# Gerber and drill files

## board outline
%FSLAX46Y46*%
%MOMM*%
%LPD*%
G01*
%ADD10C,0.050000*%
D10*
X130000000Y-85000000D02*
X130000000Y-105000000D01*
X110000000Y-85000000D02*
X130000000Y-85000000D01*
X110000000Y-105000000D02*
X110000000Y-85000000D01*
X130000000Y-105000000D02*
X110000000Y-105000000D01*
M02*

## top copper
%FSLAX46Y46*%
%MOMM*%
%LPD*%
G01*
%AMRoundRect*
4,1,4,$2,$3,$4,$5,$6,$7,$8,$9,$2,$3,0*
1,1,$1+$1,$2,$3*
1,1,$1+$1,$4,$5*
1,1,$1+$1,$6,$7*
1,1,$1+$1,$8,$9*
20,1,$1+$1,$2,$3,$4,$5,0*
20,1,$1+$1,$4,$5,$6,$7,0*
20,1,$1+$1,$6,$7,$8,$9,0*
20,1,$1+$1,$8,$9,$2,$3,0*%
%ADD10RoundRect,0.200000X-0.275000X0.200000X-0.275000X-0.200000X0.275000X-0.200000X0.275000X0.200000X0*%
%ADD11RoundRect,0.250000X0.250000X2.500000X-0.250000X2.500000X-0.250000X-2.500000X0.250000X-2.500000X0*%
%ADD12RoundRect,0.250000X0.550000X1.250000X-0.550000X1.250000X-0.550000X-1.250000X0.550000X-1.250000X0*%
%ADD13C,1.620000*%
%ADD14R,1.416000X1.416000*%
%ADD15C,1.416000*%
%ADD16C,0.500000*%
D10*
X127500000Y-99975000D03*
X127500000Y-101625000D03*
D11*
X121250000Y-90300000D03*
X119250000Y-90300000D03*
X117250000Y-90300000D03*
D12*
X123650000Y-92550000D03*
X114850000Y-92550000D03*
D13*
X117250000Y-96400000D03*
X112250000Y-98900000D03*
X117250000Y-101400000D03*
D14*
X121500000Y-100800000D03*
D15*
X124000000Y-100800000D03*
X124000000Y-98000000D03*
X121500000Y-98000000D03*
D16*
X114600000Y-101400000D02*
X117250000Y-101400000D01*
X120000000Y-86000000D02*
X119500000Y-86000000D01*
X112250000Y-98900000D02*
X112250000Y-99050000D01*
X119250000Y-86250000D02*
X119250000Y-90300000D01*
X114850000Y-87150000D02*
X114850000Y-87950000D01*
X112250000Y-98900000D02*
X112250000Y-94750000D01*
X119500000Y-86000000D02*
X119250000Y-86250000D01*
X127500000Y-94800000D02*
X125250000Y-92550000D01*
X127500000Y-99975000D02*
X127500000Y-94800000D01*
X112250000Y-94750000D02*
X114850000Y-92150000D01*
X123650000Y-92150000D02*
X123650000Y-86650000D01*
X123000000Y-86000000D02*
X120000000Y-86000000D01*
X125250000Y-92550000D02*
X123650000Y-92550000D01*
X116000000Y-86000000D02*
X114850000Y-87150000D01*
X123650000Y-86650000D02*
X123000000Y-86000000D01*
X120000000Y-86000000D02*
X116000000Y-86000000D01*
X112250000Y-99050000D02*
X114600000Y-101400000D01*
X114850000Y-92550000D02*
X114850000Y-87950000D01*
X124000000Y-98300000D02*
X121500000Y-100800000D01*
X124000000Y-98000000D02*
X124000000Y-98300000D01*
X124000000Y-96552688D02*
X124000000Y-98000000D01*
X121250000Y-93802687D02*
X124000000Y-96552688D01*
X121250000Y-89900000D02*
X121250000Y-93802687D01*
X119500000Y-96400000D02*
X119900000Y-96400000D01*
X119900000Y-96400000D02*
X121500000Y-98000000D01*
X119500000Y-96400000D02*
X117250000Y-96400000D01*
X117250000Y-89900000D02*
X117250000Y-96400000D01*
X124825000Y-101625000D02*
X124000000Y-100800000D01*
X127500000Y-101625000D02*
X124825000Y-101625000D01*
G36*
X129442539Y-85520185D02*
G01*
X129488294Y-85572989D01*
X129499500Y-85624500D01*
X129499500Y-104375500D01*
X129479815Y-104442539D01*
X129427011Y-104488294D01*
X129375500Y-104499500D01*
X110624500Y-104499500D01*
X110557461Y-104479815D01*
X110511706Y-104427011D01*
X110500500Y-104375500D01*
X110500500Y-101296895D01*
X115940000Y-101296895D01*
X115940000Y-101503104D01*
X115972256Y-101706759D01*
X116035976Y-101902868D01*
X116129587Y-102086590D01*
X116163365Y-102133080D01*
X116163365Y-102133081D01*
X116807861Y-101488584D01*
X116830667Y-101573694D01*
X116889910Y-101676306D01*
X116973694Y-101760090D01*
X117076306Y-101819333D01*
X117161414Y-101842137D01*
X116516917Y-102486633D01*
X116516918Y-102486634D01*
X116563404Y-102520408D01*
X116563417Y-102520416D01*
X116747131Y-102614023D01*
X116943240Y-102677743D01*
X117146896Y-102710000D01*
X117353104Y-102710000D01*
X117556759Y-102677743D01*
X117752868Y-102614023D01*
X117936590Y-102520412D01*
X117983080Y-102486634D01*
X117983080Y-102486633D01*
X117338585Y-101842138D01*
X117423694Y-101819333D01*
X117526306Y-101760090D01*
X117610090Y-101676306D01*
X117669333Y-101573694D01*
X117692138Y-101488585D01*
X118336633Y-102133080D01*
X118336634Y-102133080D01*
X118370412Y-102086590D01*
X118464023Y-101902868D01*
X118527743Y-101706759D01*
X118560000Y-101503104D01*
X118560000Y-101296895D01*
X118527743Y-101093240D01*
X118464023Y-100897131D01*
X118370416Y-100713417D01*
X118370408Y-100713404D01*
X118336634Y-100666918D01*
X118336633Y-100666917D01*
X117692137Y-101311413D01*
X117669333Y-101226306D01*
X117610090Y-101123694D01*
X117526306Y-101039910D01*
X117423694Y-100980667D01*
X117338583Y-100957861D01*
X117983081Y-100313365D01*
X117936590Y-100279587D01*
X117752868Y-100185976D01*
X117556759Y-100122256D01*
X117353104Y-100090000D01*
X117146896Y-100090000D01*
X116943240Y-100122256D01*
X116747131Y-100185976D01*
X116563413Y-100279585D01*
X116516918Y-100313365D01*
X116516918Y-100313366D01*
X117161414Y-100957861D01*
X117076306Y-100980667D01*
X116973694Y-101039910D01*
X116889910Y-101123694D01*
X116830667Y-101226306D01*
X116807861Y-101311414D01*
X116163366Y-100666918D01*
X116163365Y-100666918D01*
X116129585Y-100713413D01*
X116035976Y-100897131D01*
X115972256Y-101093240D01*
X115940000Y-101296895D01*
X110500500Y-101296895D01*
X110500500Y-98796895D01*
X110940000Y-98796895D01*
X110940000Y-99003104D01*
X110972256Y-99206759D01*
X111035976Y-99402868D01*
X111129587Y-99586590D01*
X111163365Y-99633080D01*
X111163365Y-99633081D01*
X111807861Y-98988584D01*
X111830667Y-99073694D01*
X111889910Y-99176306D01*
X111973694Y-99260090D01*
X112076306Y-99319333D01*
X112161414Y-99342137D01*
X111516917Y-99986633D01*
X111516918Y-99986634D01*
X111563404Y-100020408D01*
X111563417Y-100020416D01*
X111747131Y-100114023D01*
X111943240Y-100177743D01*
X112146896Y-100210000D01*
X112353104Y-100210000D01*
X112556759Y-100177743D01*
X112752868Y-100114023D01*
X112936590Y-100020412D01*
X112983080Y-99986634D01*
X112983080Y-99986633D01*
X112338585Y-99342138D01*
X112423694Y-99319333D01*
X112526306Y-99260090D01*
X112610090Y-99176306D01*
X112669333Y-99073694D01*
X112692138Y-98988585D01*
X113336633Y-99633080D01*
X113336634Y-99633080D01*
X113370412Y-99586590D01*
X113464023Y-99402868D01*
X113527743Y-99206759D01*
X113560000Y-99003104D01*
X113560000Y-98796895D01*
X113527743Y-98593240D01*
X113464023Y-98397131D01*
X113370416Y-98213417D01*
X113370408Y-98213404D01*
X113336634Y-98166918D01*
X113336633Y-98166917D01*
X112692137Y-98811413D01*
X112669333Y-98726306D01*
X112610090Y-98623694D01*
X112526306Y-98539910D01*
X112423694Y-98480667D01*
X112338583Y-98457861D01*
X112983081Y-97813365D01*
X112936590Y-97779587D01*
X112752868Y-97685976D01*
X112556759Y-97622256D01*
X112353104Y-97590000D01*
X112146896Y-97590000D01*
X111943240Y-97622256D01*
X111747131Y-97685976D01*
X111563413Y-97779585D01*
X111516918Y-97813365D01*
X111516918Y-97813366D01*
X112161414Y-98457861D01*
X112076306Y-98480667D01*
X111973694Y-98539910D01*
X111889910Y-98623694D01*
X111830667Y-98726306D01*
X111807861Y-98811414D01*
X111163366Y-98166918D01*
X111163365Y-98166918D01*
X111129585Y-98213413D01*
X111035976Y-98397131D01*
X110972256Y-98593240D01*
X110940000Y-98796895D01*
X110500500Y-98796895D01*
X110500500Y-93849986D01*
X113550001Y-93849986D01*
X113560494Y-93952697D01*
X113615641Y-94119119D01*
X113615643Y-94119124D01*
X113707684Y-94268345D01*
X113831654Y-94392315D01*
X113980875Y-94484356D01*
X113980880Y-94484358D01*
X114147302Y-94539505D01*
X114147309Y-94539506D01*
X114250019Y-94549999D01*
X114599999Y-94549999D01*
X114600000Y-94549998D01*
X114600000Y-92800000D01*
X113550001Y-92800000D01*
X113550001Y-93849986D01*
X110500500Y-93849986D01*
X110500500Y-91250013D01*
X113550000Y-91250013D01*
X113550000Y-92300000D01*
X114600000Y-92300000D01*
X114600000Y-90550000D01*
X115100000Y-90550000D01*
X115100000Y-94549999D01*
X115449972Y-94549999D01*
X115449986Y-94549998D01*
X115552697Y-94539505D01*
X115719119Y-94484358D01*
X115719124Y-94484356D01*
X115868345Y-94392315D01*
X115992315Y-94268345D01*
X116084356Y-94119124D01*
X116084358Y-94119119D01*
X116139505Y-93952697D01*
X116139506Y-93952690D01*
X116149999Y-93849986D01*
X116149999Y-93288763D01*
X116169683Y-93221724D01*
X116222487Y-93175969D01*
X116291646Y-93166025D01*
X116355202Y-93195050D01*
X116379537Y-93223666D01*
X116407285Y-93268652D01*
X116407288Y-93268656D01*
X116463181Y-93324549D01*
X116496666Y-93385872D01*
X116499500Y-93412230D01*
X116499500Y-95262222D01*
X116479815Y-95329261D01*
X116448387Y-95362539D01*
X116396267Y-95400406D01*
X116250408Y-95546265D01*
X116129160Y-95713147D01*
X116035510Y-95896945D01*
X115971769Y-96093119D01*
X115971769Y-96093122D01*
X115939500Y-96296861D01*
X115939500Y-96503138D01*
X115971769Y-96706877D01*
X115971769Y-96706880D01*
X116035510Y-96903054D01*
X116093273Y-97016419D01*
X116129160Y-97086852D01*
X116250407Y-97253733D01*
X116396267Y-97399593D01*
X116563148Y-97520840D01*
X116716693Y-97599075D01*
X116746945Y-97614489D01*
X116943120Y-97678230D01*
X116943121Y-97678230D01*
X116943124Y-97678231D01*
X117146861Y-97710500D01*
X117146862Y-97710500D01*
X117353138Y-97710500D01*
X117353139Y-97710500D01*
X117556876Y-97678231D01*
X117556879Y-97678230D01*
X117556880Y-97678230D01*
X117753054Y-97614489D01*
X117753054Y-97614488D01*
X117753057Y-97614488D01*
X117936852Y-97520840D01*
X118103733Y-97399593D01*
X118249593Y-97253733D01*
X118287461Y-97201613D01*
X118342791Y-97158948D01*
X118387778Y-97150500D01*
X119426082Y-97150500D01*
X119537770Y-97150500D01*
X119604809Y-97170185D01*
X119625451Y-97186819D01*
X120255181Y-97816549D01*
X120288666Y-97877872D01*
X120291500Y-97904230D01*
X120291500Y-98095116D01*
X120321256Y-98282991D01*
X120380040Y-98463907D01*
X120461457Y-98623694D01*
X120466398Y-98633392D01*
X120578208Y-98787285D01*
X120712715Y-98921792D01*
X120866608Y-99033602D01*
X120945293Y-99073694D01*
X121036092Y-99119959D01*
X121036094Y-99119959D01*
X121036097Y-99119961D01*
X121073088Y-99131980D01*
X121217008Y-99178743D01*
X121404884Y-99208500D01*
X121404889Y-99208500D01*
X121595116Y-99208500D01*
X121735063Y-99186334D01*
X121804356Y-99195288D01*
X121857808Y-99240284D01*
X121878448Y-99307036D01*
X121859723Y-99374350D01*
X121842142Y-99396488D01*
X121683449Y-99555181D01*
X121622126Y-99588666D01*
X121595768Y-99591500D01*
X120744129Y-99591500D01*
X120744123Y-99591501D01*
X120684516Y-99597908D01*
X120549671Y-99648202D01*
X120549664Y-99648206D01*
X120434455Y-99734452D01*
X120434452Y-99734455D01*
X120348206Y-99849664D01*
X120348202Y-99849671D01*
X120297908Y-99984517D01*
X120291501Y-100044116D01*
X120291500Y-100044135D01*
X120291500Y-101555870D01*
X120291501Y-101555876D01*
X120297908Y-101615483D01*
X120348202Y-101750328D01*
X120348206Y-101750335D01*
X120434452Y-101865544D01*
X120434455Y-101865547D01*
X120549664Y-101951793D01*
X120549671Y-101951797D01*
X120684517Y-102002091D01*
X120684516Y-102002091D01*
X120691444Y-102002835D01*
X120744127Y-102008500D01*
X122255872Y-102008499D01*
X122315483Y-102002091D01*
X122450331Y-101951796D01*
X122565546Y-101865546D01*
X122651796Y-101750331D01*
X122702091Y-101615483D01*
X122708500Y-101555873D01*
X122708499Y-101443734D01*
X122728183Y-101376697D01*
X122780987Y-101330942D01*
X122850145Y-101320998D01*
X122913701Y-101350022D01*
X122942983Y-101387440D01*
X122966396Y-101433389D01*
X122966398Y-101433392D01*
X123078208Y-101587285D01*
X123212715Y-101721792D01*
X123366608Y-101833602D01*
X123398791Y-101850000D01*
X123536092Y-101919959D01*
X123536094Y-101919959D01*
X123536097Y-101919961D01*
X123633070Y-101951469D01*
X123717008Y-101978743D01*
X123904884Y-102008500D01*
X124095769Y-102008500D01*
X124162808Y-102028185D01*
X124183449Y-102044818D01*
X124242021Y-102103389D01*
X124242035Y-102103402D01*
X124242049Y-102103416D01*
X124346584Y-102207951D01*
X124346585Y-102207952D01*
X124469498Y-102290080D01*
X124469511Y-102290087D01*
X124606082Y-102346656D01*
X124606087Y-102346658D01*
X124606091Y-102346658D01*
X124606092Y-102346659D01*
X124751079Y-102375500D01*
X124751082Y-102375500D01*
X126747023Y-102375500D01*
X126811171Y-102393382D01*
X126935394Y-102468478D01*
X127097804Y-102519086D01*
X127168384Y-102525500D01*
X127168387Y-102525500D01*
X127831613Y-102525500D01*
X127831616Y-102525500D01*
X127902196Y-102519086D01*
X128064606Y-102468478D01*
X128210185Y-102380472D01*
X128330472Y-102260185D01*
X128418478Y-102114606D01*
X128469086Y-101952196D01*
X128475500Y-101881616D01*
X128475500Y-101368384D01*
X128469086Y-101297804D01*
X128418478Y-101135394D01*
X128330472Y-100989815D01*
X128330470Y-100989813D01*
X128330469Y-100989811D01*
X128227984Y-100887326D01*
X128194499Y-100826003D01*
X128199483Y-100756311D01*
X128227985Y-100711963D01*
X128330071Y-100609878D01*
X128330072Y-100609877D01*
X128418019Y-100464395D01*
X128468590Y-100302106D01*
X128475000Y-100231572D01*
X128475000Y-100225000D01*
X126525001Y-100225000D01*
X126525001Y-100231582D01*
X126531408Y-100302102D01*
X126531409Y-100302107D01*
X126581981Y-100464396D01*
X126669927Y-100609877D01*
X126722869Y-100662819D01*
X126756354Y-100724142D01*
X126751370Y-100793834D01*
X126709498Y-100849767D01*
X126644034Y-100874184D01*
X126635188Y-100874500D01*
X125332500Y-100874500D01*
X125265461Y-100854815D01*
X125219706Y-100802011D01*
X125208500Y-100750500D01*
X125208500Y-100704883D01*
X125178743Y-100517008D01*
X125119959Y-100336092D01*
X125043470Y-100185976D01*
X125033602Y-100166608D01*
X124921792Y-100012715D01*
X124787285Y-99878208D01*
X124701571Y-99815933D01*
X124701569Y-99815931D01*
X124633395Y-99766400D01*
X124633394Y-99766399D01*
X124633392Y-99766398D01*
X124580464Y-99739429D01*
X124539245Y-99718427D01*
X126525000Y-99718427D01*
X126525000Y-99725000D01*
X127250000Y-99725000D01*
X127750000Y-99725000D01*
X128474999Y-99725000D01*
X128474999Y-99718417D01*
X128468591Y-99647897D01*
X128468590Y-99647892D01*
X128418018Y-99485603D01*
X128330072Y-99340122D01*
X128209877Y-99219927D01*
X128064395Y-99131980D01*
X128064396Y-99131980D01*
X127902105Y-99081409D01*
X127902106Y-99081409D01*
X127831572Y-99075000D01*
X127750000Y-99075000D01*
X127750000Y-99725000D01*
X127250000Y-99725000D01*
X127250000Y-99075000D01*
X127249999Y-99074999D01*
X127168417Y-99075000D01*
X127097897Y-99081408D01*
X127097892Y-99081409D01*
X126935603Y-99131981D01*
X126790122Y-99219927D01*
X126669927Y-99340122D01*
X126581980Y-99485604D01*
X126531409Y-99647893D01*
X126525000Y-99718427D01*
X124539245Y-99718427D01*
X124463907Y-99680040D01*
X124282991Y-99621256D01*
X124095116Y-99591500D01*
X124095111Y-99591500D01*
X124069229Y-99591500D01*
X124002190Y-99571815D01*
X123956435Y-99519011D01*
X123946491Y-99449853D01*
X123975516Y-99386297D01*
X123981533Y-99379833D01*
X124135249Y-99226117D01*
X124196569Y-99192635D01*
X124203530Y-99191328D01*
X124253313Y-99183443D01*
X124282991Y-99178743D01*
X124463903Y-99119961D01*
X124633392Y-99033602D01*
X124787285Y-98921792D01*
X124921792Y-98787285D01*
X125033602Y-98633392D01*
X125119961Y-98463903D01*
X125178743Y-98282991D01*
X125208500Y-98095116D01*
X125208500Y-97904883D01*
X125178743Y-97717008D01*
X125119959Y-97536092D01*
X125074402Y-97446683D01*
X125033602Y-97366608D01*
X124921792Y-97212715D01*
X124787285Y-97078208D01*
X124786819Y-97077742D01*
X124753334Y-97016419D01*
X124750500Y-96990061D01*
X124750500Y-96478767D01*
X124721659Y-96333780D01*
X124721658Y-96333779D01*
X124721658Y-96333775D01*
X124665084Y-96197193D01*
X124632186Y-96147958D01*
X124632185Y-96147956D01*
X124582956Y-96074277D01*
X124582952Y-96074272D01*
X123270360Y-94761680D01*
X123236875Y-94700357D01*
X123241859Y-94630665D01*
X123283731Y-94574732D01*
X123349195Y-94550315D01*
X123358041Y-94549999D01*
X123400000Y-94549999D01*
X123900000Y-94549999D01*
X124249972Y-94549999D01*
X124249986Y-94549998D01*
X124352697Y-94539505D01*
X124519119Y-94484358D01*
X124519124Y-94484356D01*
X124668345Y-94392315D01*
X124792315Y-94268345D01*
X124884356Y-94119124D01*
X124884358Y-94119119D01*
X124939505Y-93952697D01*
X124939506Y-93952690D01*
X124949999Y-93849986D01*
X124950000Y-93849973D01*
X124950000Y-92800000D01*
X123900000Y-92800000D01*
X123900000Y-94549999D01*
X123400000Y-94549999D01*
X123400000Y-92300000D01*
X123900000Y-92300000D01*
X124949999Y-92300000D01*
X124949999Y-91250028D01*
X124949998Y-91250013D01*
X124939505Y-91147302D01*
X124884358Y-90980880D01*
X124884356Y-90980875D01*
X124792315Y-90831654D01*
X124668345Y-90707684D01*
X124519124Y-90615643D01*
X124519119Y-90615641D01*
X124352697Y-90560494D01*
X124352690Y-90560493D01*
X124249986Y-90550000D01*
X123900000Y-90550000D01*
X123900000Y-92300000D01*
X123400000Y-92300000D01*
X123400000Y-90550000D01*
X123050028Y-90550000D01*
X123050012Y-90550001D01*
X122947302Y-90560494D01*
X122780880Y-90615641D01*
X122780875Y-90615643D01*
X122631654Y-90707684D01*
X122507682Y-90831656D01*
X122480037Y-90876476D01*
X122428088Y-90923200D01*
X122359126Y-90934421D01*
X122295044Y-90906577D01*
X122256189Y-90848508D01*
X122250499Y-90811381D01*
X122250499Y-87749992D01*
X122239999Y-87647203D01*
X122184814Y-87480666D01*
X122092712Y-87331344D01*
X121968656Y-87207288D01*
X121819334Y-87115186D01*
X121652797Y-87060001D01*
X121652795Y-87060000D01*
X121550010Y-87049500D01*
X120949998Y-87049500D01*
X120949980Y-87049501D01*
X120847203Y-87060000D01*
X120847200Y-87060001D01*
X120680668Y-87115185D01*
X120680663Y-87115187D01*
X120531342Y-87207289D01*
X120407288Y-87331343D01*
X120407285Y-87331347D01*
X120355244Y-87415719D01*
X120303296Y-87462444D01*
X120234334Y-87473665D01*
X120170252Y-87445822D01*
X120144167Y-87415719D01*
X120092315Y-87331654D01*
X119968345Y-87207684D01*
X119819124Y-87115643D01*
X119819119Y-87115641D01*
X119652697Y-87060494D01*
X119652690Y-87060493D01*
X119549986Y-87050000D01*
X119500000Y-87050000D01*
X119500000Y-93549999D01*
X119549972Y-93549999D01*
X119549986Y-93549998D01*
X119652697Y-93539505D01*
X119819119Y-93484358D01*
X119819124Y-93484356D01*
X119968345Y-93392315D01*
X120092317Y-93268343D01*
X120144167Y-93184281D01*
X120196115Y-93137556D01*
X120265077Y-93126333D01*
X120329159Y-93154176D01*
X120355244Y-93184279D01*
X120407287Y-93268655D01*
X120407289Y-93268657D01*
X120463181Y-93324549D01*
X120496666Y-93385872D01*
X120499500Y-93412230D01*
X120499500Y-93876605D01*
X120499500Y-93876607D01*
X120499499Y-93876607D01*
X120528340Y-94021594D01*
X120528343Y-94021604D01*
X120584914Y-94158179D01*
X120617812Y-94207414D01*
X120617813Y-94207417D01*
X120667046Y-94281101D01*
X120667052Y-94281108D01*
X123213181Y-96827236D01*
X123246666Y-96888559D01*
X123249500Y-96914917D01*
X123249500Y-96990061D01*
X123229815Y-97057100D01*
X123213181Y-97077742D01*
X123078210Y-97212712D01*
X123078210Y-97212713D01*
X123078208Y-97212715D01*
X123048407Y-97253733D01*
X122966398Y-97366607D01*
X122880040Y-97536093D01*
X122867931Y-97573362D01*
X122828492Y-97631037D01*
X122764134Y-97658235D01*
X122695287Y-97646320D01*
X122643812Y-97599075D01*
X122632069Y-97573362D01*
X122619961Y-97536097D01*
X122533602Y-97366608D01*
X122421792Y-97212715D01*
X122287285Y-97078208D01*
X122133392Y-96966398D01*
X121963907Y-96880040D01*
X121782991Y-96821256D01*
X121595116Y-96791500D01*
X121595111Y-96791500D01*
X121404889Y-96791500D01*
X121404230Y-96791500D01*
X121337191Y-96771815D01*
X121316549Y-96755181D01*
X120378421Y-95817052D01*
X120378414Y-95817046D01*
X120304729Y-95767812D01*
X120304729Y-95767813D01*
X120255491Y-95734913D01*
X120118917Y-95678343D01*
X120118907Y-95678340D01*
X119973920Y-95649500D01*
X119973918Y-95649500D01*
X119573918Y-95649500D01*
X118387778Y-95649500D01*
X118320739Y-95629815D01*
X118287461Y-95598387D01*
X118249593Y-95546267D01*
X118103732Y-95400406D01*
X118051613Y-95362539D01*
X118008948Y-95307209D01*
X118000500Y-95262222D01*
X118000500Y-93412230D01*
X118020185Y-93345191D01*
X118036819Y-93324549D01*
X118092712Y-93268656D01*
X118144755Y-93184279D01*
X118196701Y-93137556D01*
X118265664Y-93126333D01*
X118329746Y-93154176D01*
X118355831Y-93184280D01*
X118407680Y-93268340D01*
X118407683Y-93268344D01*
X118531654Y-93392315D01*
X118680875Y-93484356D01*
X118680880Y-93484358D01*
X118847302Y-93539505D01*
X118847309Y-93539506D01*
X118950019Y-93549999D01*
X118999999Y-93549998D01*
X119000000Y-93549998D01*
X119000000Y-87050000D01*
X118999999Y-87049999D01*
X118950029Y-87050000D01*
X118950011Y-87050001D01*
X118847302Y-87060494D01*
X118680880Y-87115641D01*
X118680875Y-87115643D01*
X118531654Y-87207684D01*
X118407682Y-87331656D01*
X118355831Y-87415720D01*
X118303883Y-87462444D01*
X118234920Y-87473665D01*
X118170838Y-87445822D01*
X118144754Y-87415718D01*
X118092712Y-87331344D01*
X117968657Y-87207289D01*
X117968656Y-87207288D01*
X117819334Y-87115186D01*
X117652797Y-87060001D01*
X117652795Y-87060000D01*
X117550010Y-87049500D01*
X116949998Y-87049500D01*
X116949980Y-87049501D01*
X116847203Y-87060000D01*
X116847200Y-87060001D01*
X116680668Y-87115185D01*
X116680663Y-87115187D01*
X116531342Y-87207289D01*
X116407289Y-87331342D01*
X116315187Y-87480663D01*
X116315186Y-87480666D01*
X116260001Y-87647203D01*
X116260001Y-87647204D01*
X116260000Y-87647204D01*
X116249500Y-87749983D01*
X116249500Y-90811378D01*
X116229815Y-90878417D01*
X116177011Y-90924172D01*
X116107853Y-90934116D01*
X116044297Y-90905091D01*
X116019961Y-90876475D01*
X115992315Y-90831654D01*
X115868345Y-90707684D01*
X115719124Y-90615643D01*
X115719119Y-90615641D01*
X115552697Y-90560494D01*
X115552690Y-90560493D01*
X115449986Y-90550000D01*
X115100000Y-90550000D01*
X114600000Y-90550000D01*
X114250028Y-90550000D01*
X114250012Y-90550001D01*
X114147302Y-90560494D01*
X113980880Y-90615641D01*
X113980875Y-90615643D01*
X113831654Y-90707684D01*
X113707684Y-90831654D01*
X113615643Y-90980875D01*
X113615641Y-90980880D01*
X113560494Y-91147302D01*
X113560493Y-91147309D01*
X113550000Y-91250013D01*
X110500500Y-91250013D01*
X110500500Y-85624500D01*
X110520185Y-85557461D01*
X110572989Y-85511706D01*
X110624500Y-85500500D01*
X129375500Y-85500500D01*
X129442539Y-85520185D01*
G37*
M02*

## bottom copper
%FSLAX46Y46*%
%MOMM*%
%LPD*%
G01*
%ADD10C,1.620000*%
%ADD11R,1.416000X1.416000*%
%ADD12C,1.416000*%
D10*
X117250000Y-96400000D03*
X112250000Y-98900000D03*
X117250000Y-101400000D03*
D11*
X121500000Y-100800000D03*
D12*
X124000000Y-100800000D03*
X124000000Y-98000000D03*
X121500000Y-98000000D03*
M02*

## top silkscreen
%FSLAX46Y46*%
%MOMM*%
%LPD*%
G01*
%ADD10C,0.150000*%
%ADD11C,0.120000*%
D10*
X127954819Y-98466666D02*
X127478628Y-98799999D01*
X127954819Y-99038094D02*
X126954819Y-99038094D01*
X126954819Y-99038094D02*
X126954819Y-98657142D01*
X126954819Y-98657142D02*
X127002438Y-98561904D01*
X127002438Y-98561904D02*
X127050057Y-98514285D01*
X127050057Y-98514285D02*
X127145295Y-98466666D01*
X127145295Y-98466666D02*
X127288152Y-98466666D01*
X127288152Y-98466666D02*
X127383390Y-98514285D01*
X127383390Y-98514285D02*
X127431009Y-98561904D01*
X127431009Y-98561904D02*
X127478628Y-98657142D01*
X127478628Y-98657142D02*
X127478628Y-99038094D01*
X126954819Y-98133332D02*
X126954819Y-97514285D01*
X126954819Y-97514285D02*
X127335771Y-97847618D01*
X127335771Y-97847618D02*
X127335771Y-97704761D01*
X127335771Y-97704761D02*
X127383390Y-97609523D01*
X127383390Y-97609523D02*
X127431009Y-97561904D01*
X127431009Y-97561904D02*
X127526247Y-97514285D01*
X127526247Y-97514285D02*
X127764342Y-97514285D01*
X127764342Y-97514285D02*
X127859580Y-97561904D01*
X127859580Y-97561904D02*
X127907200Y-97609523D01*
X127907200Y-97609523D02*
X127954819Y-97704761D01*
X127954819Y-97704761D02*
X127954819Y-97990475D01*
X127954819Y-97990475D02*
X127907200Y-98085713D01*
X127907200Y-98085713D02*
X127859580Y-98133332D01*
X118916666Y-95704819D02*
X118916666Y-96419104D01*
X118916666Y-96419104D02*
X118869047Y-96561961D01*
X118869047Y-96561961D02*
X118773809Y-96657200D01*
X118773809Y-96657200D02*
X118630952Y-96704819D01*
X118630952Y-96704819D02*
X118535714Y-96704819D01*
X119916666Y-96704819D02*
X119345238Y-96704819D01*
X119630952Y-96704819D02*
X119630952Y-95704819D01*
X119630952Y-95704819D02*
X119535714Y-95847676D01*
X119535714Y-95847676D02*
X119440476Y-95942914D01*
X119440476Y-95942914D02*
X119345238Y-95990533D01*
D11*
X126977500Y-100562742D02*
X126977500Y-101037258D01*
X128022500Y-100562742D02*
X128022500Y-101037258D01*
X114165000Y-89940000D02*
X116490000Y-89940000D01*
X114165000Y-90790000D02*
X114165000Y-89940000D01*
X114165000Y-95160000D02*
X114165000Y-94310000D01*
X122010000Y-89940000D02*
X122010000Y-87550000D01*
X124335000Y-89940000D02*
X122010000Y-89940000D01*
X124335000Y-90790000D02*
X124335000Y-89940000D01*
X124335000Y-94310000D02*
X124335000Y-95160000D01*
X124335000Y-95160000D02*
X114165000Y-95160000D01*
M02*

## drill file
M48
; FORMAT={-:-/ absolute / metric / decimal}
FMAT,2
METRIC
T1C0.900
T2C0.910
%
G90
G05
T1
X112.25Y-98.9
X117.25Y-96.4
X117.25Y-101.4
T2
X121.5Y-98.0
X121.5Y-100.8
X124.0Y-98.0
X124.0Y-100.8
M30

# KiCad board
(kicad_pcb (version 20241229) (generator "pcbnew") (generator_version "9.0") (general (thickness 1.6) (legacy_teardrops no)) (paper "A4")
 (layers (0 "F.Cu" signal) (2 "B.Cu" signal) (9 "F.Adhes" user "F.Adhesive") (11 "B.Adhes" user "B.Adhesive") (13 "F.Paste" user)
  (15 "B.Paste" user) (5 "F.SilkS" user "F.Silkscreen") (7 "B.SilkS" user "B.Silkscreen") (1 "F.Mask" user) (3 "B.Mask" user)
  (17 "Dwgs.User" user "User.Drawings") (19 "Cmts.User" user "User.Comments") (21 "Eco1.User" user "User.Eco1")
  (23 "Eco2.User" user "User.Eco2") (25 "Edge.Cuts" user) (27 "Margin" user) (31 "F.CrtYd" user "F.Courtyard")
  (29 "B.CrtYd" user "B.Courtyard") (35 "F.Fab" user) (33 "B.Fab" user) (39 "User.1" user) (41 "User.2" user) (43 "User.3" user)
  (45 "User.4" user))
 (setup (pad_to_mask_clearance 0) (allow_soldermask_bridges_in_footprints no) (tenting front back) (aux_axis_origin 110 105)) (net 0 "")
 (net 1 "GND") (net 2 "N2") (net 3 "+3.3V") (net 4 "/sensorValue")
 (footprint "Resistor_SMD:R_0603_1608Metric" (layer "F.Cu") (at 127.5 100.8 -90)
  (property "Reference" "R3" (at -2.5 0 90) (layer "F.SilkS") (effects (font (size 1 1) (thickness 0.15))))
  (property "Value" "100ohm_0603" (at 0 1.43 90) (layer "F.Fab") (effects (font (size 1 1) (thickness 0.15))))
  (fp_line (start -0.237258 0.5225) (end 0.237258 0.5225) (stroke (width 0.12) (type solid)) (layer "F.SilkS"))
  (fp_line (start -0.237258 -0.5225) (end 0.237258 -0.5225) (stroke (width 0.12) (type solid)) (layer "F.SilkS"))
  (pad "1" smd roundrect (at -0.825 0 270) (size 0.8 0.95) (layers "F.Cu" "F.Mask" "F.Paste") (roundrect_rratio 0.25) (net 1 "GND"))
  (pad "2" smd roundrect (at 0.825 0 270) (size 0.8 0.95) (layers "F.Cu" "F.Mask" "F.Paste") (roundrect_rratio 0.25) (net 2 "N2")))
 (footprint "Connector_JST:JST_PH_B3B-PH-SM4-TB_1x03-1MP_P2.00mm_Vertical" (layer "F.Cu") (at 119.25 90.8 180)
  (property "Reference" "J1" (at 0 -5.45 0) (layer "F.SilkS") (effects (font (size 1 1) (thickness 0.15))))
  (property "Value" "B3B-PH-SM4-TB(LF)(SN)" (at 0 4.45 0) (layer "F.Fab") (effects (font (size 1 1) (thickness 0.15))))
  (fp_line (start 5.085 0.86) (end 2.76 0.86) (stroke (width 0.12) (type solid)) (layer "F.SilkS"))
  (fp_line (start 5.085 0.01) (end 5.085 0.86) (stroke (width 0.12) (type solid)) (layer "F.SilkS"))
  (fp_line (start 5.085 -4.36) (end 5.085 -3.51) (stroke (width 0.12) (type solid)) (layer "F.SilkS"))
  (fp_line (start -2.76 0.86) (end -2.76 3.25) (stroke (width 0.12) (type solid)) (layer "F.SilkS"))
  (fp_line (start -5.085 0.86) (end -2.76 0.86) (stroke (width 0.12) (type solid)) (layer "F.SilkS"))
  (fp_line (start -5.085 0.01) (end -5.085 0.86) (stroke (width 0.12) (type solid)) (layer "F.SilkS"))
  (fp_line (start -5.085 -3.51) (end -5.085 -4.36) (stroke (width 0.12) (type solid)) (layer "F.SilkS"))
  (fp_line (start -5.085 -4.36) (end 5.085 -4.36) (stroke (width 0.12) (type solid)) (layer "F.SilkS"))
  (pad "1" smd roundrect (at -2 0.5 180) (size 1 5.5) (layers "F.Cu" "F.Mask" "F.Paste") (roundrect_rratio 0.25) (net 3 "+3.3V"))
  (pad "2" smd roundrect (at 0 0.5 180) (size 1 5.5) (layers "F.Cu" "F.Mask" "F.Paste") (roundrect_rratio 0.25) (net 1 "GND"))
  (pad "3" smd roundrect (at 2 0.5 180) (size 1 5.5) (layers "F.Cu" "F.Mask" "F.Paste") (roundrect_rratio 0.25) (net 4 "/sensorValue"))
  (pad "MP" smd roundrect (at -4.4 -1.75 180) (size 1.6 3) (layers "F.Cu" "F.Mask" "F.Paste") (roundrect_rratio 0.15625) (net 1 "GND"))
  (pad "MP" smd roundrect (at 4.4 -1.75 180) (size 1.6 3) (layers "F.Cu" "F.Mask" "F.Paste") (roundrect_rratio 0.15625) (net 1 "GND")))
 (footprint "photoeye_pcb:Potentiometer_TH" (layer "B.Cu") (at 117.25 96.4 180)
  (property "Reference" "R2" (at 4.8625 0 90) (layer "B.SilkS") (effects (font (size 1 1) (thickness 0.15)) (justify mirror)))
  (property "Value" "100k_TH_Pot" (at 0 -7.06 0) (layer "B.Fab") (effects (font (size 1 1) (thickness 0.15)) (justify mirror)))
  (pad "1" thru_hole circle (at 0 0 180) (size 1.62 1.62) (drill 0.9) (layers "*.Cu" "*.Mask") (remove_unused_layers no)
   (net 4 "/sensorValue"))
  (pad "2" thru_hole circle (at 5 -2.5 180) (size 1.62 1.62) (drill 0.9) (layers "*.Cu" "*.Mask") (remove_unused_layers no) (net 1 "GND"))
  (pad "3" thru_hole circle (at 0 -5 180) (size 1.62 1.62) (drill 0.9) (layers "*.Cu" "*.Mask") (remove_unused_layers no) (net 1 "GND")))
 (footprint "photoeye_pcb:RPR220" (layer "B.Cu") (at 121.5 100.8 90)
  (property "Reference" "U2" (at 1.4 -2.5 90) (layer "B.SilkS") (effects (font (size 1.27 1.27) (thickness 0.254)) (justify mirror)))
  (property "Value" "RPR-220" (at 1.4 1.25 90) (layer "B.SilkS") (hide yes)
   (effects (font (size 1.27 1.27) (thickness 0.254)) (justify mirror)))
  (pad "1" thru_hole rect (at 0 0 90) (size 1.416 1.416) (drill 0.91) (layers "*.Cu" "*.Mask") (remove_unused_layers no) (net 3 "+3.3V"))
  (pad "2" thru_hole circle (at 0 2.5 90) (size 1.416 1.416) (drill 0.91) (layers "*.Cu" "*.Mask") (remove_unused_layers no) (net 2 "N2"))
  (pad "3" thru_hole circle (at 2.8 2.5 90) (size 1.416 1.416) (drill 0.91) (layers "*.Cu" "*.Mask") (remove_unused_layers no)
   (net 3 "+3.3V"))
  (pad "4" thru_hole circle (at 2.8 0 90) (size 1.416 1.416) (drill 0.91) (layers "*.Cu" "*.Mask") (remove_unused_layers no)
   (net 4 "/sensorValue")))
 (gr_line (start 130 85) (end 130 105) (stroke (width 0.05) (type default)) (layer "Edge.Cuts"))
 (gr_line (start 110 85) (end 130 85) (stroke (width 0.05) (type default)) (layer "Edge.Cuts"))
 (gr_line (start 110 105) (end 110 85) (stroke (width 0.05) (type solid)) (layer "Edge.Cuts"))
 (gr_line (start 130 105) (end 110 105) (stroke (width 0.05) (type default)) (layer "Edge.Cuts"))
 (segment (start 114.6 101.4) (end 117.25 101.4) (width 0.5) (layer "F.Cu") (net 1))
 (segment (start 120 86) (end 119.5 86) (width 0.5) (layer "F.Cu") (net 1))
 (segment (start 112.25 98.9) (end 112.25 99.05) (width 0.5) (layer "F.Cu") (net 1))
 (segment (start 119.25 86.25) (end 119.25 90.3) (width 0.5) (layer "F.Cu") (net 1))
 (segment (start 114.85 87.15) (end 114.85 87.95) (width 0.5) (layer "F.Cu") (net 1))
 (segment (start 112.25 98.9) (end 112.25 94.75) (width 0.5) (layer "F.Cu") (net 1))
 (segment (start 119.5 86) (end 119.25 86.25) (width 0.5) (layer "F.Cu") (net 1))
 (segment (start 127.5 94.8) (end 125.25 92.55) (width 0.5) (layer "F.Cu") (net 1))
 (segment (start 127.5 99.975) (end 127.5 94.8) (width 0.5) (layer "F.Cu") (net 1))
 (segment (start 112.25 94.75) (end 114.85 92.15) (width 0.5) (layer "F.Cu") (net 1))
 (segment (start 123.65 92.15) (end 123.65 86.65) (width 0.5) (layer "F.Cu") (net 1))
 (segment (start 123 86) (end 120 86) (width 0.5) (layer "F.Cu") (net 1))
 (segment (start 125.25 92.55) (end 123.65 92.55) (width 0.5) (layer "F.Cu") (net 1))
 (segment (start 116 86) (end 114.85 87.15) (width 0.5) (layer "F.Cu") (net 1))
 (segment (start 123.65 86.65) (end 123 86) (width 0.5) (layer "F.Cu") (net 1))
 (segment (start 120 86) (end 116 86) (width 0.5) (layer "F.Cu") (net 1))
 (segment (start 112.25 99.05) (end 114.6 101.4) (width 0.5) (layer "F.Cu") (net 1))
 (segment (start 114.85 92.55) (end 114.85 87.95) (width 0.5) (layer "F.Cu") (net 1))
 (segment (start 124 98.3) (end 121.5 100.8) (width 0.5) (layer "F.Cu") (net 3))
 (segment (start 124 98) (end 124 98.3) (width 0.5) (layer "F.Cu") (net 3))
 (segment (start 124 96.552688) (end 124 98) (width 0.5) (layer "F.Cu") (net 3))
 (segment (start 121.25 93.802687) (end 124 96.552688) (width 0.5) (layer "F.Cu") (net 3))
 (segment (start 121.25 89.9) (end 121.25 93.802687) (width 0.5) (layer "F.Cu") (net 3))
 (segment (start 119.5 96.4) (end 119.9 96.4) (width 0.5) (layer "F.Cu") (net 4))
 (segment (start 119.9 96.4) (end 121.5 98) (width 0.5) (layer "F.Cu") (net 4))
 (segment (start 119.5 96.4) (end 117.25 96.4) (width 0.5) (layer "F.Cu") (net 4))
 (segment (start 117.25 89.9) (end 117.25 96.4) (width 0.5) (layer "F.Cu") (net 4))
 (segment (start 124.825 101.625) (end 124 100.8) (width 0.5) (layer "F.Cu") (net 2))
 (segment (start 127.5 101.625) (end 124.825 101.625) (width 0.5) (layer "F.Cu") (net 2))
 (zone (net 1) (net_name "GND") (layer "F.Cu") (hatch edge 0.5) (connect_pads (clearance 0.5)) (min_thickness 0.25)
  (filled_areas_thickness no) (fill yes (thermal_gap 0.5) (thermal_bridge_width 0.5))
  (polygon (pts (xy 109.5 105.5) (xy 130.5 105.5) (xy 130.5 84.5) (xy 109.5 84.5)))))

